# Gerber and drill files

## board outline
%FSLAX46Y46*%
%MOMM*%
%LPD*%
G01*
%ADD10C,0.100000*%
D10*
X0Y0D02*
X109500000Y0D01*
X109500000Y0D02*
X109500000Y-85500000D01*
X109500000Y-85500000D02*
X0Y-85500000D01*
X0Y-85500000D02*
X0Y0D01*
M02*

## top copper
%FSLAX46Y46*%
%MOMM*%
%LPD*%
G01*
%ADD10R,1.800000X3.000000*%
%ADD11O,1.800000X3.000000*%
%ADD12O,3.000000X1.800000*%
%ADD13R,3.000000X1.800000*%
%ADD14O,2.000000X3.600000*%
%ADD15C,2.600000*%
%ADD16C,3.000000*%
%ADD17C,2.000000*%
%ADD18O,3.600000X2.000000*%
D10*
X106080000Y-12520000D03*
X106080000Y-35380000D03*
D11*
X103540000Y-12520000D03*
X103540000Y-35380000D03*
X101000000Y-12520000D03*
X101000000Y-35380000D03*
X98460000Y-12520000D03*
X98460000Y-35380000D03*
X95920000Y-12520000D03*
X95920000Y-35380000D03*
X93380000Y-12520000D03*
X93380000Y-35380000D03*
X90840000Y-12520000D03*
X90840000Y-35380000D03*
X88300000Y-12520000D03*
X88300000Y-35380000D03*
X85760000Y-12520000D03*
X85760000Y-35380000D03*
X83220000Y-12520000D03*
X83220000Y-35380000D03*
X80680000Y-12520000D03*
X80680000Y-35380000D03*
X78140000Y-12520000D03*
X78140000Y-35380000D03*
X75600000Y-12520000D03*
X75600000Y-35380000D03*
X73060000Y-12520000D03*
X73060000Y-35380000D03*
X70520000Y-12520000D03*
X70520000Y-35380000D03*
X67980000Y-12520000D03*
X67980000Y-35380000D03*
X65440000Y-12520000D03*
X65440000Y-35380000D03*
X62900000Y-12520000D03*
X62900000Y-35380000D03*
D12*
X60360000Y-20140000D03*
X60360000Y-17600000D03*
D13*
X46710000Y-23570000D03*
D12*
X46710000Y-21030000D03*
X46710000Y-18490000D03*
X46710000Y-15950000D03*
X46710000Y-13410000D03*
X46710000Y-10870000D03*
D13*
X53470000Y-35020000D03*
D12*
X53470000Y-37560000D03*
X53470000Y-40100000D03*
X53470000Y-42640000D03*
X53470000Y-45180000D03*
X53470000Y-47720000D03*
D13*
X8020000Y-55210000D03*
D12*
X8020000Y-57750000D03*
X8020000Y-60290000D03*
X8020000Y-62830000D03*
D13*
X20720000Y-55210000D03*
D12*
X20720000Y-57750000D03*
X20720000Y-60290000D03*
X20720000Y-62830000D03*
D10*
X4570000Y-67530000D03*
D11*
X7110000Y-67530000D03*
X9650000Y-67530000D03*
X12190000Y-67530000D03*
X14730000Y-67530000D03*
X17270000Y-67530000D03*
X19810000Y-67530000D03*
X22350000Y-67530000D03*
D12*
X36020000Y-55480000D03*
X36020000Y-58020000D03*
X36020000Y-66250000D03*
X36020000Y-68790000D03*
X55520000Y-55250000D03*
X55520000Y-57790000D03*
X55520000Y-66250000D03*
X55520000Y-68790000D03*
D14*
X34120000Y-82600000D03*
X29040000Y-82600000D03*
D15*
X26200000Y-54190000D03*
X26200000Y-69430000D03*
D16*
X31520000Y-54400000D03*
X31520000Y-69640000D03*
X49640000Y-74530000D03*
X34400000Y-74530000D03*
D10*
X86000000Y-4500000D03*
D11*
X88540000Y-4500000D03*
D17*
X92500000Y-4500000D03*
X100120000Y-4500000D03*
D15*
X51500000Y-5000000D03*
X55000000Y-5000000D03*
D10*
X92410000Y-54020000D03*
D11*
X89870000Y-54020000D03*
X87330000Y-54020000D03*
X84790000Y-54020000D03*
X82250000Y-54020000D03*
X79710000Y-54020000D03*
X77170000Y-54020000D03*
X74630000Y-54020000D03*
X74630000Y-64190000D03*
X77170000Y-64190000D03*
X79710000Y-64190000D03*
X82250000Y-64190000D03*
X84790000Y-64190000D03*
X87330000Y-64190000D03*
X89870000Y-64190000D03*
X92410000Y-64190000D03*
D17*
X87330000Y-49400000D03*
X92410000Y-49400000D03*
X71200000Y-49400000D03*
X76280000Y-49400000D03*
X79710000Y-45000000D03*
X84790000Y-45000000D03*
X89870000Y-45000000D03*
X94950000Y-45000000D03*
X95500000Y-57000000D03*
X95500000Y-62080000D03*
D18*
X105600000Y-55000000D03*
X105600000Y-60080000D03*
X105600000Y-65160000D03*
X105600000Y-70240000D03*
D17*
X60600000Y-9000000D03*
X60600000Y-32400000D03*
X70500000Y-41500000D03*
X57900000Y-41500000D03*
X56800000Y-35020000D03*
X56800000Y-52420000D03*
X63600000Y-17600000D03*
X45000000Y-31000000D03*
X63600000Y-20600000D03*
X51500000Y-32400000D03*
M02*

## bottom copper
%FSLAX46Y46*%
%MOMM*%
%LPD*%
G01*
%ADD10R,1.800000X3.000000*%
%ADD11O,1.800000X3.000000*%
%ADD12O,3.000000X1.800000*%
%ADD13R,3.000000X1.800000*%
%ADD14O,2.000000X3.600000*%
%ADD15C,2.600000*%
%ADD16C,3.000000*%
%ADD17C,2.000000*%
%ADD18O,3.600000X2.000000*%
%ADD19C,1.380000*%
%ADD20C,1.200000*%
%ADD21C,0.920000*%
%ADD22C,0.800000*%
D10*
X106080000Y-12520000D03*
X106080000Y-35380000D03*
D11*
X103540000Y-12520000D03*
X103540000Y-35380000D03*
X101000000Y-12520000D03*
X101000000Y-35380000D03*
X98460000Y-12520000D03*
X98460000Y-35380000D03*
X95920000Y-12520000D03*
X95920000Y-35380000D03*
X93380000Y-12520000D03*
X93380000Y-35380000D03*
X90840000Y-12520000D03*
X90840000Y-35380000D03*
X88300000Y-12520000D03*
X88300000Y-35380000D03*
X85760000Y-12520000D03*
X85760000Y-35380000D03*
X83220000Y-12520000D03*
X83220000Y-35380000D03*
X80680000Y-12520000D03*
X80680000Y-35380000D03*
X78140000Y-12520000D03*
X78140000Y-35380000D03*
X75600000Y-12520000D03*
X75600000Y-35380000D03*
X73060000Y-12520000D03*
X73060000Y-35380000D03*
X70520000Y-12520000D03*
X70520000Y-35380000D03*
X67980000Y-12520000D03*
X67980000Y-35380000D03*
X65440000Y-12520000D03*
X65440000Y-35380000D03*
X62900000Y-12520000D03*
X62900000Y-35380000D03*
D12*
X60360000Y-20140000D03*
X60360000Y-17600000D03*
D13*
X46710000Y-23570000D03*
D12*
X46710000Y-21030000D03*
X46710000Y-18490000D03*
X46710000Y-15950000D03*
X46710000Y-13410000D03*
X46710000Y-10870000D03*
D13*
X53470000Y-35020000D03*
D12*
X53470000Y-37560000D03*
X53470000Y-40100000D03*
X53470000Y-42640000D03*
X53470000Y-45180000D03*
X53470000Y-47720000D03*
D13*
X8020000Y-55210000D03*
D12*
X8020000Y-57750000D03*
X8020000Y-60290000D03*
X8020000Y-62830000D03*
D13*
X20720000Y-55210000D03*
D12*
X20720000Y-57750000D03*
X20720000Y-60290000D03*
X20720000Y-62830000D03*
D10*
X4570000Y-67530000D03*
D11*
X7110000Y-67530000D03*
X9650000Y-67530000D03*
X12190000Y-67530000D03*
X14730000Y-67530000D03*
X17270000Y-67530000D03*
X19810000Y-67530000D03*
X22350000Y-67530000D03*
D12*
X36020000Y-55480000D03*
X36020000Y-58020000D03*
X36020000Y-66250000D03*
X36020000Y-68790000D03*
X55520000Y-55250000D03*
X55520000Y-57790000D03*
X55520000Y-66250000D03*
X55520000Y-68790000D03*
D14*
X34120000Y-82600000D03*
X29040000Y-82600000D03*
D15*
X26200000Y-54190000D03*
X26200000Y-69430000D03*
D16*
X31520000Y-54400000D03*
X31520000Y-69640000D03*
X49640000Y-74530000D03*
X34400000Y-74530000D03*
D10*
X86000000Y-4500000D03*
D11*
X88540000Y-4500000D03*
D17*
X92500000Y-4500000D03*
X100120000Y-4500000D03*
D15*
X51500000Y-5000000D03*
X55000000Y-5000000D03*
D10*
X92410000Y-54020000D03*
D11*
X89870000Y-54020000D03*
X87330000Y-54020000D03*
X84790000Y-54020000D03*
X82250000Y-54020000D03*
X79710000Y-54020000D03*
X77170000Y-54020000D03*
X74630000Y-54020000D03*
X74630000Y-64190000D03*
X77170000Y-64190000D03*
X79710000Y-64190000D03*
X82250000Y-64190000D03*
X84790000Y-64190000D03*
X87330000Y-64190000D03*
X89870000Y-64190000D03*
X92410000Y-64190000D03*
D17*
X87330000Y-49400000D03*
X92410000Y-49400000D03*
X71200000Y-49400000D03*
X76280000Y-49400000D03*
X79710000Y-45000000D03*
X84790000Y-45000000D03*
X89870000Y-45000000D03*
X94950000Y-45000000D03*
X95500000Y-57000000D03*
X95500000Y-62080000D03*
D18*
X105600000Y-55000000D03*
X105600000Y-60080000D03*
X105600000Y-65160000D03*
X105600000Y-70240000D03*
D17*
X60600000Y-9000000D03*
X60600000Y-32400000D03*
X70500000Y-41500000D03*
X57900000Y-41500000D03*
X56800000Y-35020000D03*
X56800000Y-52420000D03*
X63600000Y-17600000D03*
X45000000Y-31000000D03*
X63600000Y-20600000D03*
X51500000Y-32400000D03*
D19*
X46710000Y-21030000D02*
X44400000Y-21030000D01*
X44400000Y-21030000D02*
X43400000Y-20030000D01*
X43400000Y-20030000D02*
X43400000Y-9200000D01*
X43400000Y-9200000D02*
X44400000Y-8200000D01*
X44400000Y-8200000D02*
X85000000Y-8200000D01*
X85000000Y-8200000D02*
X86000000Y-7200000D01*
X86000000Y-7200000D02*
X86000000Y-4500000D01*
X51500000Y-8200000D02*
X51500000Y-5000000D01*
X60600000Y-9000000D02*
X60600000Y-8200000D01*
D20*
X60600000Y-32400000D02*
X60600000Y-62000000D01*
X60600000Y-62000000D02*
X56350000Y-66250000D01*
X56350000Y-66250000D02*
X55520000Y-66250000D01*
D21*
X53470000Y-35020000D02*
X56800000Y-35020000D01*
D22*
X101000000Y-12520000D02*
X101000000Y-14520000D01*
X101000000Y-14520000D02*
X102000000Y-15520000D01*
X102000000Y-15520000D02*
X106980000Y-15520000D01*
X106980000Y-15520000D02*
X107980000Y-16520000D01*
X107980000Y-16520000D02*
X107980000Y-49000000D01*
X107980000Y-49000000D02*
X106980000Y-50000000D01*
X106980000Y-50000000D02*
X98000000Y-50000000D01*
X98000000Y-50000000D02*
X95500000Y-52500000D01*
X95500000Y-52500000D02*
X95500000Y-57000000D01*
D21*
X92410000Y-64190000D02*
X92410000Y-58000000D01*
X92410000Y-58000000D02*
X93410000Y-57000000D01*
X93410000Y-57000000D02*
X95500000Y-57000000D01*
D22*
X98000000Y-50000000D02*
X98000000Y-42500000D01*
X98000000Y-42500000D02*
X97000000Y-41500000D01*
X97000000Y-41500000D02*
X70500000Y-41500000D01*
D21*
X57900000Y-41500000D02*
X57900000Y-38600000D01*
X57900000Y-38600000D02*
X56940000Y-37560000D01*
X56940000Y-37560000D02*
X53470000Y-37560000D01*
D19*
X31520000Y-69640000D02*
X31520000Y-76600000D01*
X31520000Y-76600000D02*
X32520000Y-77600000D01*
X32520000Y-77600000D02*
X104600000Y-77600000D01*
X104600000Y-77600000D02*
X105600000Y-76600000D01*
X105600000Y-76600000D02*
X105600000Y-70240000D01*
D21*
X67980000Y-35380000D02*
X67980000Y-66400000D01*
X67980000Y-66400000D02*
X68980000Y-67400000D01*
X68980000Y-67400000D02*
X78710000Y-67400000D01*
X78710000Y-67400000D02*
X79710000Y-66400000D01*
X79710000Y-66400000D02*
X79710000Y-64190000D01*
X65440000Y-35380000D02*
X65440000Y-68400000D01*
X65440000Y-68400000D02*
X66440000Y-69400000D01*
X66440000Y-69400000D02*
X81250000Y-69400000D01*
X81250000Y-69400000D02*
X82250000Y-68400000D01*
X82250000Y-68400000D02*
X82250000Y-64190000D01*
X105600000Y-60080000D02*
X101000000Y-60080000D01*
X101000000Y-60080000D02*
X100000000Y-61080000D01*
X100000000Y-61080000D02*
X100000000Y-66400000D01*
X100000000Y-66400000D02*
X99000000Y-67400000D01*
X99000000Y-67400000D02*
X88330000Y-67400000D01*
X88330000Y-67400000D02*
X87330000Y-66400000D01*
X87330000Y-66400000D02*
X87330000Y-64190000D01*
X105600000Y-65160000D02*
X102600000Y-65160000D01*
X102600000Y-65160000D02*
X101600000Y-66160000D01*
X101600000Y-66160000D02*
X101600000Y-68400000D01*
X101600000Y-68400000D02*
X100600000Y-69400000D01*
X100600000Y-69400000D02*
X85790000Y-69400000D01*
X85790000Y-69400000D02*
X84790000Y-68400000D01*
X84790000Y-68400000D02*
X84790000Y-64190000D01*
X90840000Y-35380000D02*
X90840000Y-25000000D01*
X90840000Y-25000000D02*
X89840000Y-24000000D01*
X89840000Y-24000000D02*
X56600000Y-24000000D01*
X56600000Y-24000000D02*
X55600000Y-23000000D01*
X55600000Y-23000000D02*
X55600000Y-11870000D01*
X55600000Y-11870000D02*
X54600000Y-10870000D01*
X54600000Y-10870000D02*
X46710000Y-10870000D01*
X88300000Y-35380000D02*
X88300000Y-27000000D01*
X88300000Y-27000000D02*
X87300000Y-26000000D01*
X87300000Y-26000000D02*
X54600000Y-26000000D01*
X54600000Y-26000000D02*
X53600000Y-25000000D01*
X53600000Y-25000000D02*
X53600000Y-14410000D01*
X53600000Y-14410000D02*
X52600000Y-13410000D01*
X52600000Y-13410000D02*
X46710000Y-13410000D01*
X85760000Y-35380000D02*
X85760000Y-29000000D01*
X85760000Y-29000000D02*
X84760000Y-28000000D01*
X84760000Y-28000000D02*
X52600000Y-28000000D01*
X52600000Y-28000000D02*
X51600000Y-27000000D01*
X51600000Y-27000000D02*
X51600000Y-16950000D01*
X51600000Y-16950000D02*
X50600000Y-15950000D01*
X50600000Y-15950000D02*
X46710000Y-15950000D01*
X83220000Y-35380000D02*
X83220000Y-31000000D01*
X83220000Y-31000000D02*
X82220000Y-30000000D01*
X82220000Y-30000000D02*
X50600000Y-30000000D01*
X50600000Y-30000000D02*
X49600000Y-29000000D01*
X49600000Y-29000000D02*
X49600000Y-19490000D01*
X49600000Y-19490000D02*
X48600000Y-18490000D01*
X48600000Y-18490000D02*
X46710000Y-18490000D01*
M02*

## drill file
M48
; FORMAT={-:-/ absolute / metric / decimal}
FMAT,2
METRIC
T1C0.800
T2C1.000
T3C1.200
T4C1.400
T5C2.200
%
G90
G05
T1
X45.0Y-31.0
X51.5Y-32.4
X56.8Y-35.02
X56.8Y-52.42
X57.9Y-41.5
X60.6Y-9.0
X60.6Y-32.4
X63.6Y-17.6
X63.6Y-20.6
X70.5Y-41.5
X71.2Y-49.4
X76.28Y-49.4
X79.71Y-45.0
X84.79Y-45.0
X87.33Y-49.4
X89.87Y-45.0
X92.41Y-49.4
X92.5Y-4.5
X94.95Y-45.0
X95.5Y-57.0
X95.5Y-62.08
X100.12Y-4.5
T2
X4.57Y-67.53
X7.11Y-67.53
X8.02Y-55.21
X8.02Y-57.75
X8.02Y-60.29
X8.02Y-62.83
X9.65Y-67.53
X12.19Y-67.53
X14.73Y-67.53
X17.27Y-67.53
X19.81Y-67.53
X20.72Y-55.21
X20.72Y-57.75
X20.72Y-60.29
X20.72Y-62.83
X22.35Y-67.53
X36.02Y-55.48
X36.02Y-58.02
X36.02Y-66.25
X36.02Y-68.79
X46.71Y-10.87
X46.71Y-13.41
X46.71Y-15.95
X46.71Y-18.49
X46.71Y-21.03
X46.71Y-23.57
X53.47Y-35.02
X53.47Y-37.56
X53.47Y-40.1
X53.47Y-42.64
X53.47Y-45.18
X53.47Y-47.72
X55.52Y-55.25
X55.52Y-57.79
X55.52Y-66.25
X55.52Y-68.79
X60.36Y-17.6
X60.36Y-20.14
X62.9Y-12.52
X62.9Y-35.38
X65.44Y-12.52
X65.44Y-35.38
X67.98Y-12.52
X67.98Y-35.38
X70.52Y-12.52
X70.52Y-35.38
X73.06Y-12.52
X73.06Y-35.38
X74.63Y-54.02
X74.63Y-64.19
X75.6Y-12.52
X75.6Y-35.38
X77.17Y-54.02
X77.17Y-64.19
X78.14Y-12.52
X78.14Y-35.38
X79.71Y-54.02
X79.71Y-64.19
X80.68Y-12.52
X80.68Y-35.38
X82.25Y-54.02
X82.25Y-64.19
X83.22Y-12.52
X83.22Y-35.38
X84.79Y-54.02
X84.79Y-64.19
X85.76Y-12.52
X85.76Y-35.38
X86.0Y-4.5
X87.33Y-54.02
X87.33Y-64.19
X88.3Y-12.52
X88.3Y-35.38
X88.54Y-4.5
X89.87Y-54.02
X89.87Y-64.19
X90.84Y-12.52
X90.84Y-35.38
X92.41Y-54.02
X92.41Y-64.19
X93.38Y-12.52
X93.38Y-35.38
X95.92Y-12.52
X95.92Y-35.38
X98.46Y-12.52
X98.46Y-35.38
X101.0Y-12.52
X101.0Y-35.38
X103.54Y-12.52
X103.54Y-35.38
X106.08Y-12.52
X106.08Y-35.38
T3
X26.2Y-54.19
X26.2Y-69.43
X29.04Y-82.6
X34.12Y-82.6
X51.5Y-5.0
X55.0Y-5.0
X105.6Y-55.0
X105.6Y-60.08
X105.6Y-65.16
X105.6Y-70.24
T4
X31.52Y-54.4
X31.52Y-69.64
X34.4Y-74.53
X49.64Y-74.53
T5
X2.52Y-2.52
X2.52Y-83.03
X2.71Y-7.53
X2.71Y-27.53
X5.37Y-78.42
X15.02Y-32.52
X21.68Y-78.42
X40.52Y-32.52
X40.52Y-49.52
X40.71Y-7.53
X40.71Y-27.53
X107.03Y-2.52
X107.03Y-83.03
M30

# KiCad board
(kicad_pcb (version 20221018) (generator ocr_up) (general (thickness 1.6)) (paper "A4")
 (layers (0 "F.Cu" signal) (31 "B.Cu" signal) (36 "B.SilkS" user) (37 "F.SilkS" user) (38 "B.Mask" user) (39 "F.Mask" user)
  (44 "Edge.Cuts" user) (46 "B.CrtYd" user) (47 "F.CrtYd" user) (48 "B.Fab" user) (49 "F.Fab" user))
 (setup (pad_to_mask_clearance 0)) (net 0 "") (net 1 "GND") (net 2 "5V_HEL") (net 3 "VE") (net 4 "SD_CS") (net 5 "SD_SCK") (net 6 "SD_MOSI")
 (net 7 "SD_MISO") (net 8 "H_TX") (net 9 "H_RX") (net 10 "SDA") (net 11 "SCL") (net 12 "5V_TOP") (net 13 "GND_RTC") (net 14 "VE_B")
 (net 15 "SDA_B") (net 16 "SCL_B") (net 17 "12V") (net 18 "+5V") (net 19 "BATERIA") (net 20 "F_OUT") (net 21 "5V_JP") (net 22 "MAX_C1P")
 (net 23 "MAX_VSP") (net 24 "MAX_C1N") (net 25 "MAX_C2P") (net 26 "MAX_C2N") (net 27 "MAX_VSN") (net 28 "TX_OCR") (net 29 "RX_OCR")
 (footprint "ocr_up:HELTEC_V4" (layer "F.Cu") (at 106.08 12.52)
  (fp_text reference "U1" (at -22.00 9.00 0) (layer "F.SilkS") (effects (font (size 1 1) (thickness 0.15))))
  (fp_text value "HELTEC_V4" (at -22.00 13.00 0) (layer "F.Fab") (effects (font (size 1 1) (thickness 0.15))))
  (pad "A1" thru_hole rect (at -0.0 0) (size 1.8 3.0) (drill 1.0) (layers "*.Cu" "*.Mask") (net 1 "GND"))
  (pad "B1" thru_hole rect (at -0.0 22.86) (size 1.8 3.0) (drill 1.0) (layers "*.Cu" "*.Mask"))
  (pad "A2" thru_hole oval (at -2.54 0) (size 1.8 3.0) (drill 1.0) (layers "*.Cu" "*.Mask") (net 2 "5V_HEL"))
  (pad "B2" thru_hole oval (at -2.54 22.86) (size 1.8 3.0) (drill 1.0) (layers "*.Cu" "*.Mask"))
  (pad "A3" thru_hole oval (at -5.08 0) (size 1.8 3.0) (drill 1.0) (layers "*.Cu" "*.Mask") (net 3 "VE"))
  (pad "B3" thru_hole oval (at -5.08 22.86) (size 1.8 3.0) (drill 1.0) (layers "*.Cu" "*.Mask"))
  (pad "A4" thru_hole oval (at -7.62 0) (size 1.8 3.0) (drill 1.0) (layers "*.Cu" "*.Mask") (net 3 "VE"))
  (pad "B4" thru_hole oval (at -7.62 22.86) (size 1.8 3.0) (drill 1.0) (layers "*.Cu" "*.Mask"))
  (pad "A5" thru_hole oval (at -10.16 0) (size 1.8 3.0) (drill 1.0) (layers "*.Cu" "*.Mask"))
  (pad "B5" thru_hole oval (at -10.16 22.86) (size 1.8 3.0) (drill 1.0) (layers "*.Cu" "*.Mask"))
  (pad "A6" thru_hole oval (at -12.7 0) (size 1.8 3.0) (drill 1.0) (layers "*.Cu" "*.Mask"))
  (pad "B6" thru_hole oval (at -12.7 22.86) (size 1.8 3.0) (drill 1.0) (layers "*.Cu" "*.Mask"))
  (pad "A7" thru_hole oval (at -15.24 0) (size 1.8 3.0) (drill 1.0) (layers "*.Cu" "*.Mask"))
  (pad "B7" thru_hole oval (at -15.24 22.86) (size 1.8 3.0) (drill 1.0) (layers "*.Cu" "*.Mask") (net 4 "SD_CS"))
  (pad "A8" thru_hole oval (at -17.78 0) (size 1.8 3.0) (drill 1.0) (layers "*.Cu" "*.Mask"))
  (pad "B8" thru_hole oval (at -17.78 22.86) (size 1.8 3.0) (drill 1.0) (layers "*.Cu" "*.Mask") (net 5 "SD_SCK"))
  (pad "A9" thru_hole oval (at -20.32 0) (size 1.8 3.0) (drill 1.0) (layers "*.Cu" "*.Mask"))
  (pad "B9" thru_hole oval (at -20.32 22.86) (size 1.8 3.0) (drill 1.0) (layers "*.Cu" "*.Mask") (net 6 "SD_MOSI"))
  (pad "A10" thru_hole oval (at -22.86 0) (size 1.8 3.0) (drill 1.0) (layers "*.Cu" "*.Mask"))
  (pad "B10" thru_hole oval (at -22.86 22.86) (size 1.8 3.0) (drill 1.0) (layers "*.Cu" "*.Mask") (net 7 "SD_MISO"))
  (pad "A11" thru_hole oval (at -25.4 0) (size 1.8 3.0) (drill 1.0) (layers "*.Cu" "*.Mask"))
  (pad "B11" thru_hole oval (at -25.4 22.86) (size 1.8 3.0) (drill 1.0) (layers "*.Cu" "*.Mask"))
  (pad "A12" thru_hole oval (at -27.94 0) (size 1.8 3.0) (drill 1.0) (layers "*.Cu" "*.Mask"))
  (pad "B12" thru_hole oval (at -27.94 22.86) (size 1.8 3.0) (drill 1.0) (layers "*.Cu" "*.Mask"))
  (pad "A13" thru_hole oval (at -30.48 0) (size 1.8 3.0) (drill 1.0) (layers "*.Cu" "*.Mask"))
  (pad "B13" thru_hole oval (at -30.48 22.86) (size 1.8 3.0) (drill 1.0) (layers "*.Cu" "*.Mask"))
  (pad "A14" thru_hole oval (at -33.02 0) (size 1.8 3.0) (drill 1.0) (layers "*.Cu" "*.Mask"))
  (pad "B14" thru_hole oval (at -33.02 22.86) (size 1.8 3.0) (drill 1.0) (layers "*.Cu" "*.Mask"))
  (pad "A15" thru_hole oval (at -35.56 0) (size 1.8 3.0) (drill 1.0) (layers "*.Cu" "*.Mask"))
  (pad "B15" thru_hole oval (at -35.56 22.86) (size 1.8 3.0) (drill 1.0) (layers "*.Cu" "*.Mask"))
  (pad "A16" thru_hole oval (at -38.1 0) (size 1.8 3.0) (drill 1.0) (layers "*.Cu" "*.Mask"))
  (pad "B16" thru_hole oval (at -38.1 22.86) (size 1.8 3.0) (drill 1.0) (layers "*.Cu" "*.Mask") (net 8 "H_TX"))
  (pad "A17" thru_hole oval (at -40.64 0) (size 1.8 3.0) (drill 1.0) (layers "*.Cu" "*.Mask"))
  (pad "B17" thru_hole oval (at -40.64 22.86) (size 1.8 3.0) (drill 1.0) (layers "*.Cu" "*.Mask") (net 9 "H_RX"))
  (pad "A18" thru_hole oval (at -43.18 0) (size 1.8 3.0) (drill 1.0) (layers "*.Cu" "*.Mask"))
  (pad "B18" thru_hole oval (at -43.18 22.86) (size 1.8 3.0) (drill 1.0) (layers "*.Cu" "*.Mask"))
  (pad "AUX17" thru_hole oval (at -45.72 7.619999999999999) (size 3.0 1.8) (drill 1.0) (layers "*.Cu" "*.Mask") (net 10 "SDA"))
  (pad "AUX18" thru_hole oval (at -45.72 5.08) (size 3.0 1.8) (drill 1.0) (layers "*.Cu" "*.Mask") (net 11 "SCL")))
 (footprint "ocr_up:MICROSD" (layer "F.Cu") (at 0.66 5.48)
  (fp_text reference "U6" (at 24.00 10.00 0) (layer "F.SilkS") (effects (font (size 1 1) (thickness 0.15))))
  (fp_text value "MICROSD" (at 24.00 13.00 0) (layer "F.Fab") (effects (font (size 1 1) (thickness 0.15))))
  (pad "1" thru_hole rect (at 46.05 18.09) (size 3.0 1.8) (drill 1.0) (layers "*.Cu" "*.Mask") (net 1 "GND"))
  (pad "2" thru_hole oval (at 46.05 15.55) (size 3.0 1.8) (drill 1.0) (layers "*.Cu" "*.Mask") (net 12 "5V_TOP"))
  (pad "3" thru_hole oval (at 46.05 13.01) (size 3.0 1.8) (drill 1.0) (layers "*.Cu" "*.Mask") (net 7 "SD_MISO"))
  (pad "4" thru_hole oval (at 46.05 10.469999999999999) (size 3.0 1.8) (drill 1.0) (layers "*.Cu" "*.Mask") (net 6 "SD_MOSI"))
  (pad "5" thru_hole oval (at 46.05 7.93) (size 3.0 1.8) (drill 1.0) (layers "*.Cu" "*.Mask") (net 5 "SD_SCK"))
  (pad "6" thru_hole oval (at 46.05 5.390000000000001) (size 3.0 1.8) (drill 1.0) (layers "*.Cu" "*.Mask") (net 4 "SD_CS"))
  (pad "" np_thru_hole circle (at 2.05 2.05) (size 2.2 2.2) (drill 2.2) (layers "*.Cu" "*.Mask"))
  (pad "" np_thru_hole circle (at 40.05 2.05) (size 2.2 2.2) (drill 2.2) (layers "*.Cu" "*.Mask"))
  (pad "" np_thru_hole circle (at 2.05 22.05) (size 2.2 2.2) (drill 2.2) (layers "*.Cu" "*.Mask"))
  (pad "" np_thru_hole circle (at 40.05 22.05) (size 2.2 2.2) (drill 2.2) (layers "*.Cu" "*.Mask")))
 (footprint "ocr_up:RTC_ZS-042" (layer "F.Cu") (at 53.47 35.02)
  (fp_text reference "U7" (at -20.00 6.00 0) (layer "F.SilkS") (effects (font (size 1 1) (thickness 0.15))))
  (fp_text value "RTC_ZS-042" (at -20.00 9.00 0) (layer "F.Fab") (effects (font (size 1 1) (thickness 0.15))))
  (pad "1" thru_hole rect (at 0 0.0) (size 3.0 1.8) (drill 1.0) (layers "*.Cu" "*.Mask") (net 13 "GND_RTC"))
  (pad "2" thru_hole oval (at 0 2.54) (size 3.0 1.8) (drill 1.0) (layers "*.Cu" "*.Mask") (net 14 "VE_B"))
  (pad "3" thru_hole oval (at 0 5.08) (size 3.0 1.8) (drill 1.0) (layers "*.Cu" "*.Mask") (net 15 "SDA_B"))
  (pad "4" thru_hole oval (at 0 7.62) (size 3.0 1.8) (drill 1.0) (layers "*.Cu" "*.Mask") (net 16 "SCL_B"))
  (pad "5" thru_hole oval (at 0 10.16) (size 3.0 1.8) (drill 1.0) (layers "*.Cu" "*.Mask"))
  (pad "6" thru_hole oval (at 0 12.7) (size 3.0 1.8) (drill 1.0) (layers "*.Cu" "*.Mask"))
  (pad "" np_thru_hole circle (at -38.45 -2.5) (size 2.2 2.2) (drill 2.2) (layers "*.Cu" "*.Mask"))
  (pad "" np_thru_hole circle (at -12.949999999999996 -2.5) (size 2.2 2.2) (drill 2.2) (layers "*.Cu" "*.Mask"))
  (pad "" np_thru_hole circle (at -12.949999999999996 14.5) (size 2.2 2.2) (drill 2.2) (layers "*.Cu" "*.Mask")))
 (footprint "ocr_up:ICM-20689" (layer "F.Cu") (at 8.02 55.21)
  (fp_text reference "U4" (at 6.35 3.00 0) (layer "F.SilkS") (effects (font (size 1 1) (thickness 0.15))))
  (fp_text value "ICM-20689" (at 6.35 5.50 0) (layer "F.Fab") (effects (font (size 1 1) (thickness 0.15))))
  (pad "1" thru_hole rect (at 0 0.0) (size 3.0 1.8) (drill 1.0) (layers "*.Cu" "*.Mask") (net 14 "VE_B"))
  (pad "2" thru_hole oval (at 0 2.54) (size 3.0 1.8) (drill 1.0) (layers "*.Cu" "*.Mask") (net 1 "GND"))
  (pad "3" thru_hole oval (at 0 5.08) (size 3.0 1.8) (drill 1.0) (layers "*.Cu" "*.Mask") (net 16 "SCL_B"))
  (pad "4" thru_hole oval (at 0 7.62) (size 3.0 1.8) (drill 1.0) (layers "*.Cu" "*.Mask") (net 15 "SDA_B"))
  (pad "5" thru_hole rect (at 12.7 0.0) (size 3.0 1.8) (drill 1.0) (layers "*.Cu" "*.Mask"))
  (pad "6" thru_hole oval (at 12.7 2.54) (size 3.0 1.8) (drill 1.0) (layers "*.Cu" "*.Mask"))
  (pad "7" thru_hole oval (at 12.7 5.08) (size 3.0 1.8) (drill 1.0) (layers "*.Cu" "*.Mask"))
  (pad "8" thru_hole oval (at 12.7 7.62) (size 3.0 1.8) (drill 1.0) (layers "*.Cu" "*.Mask") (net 14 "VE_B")))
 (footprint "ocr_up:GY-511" (layer "F.Cu") (at 4.57 67.53)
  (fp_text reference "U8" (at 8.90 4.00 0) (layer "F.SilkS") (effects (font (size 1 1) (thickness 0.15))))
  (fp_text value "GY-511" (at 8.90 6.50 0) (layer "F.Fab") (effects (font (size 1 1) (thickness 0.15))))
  (pad "1" thru_hole rect (at 0.0 0) (size 1.8 3.0) (drill 1.0) (layers "*.Cu" "*.Mask"))
  (pad "2" thru_hole oval (at 2.54 0) (size 1.8 3.0) (drill 1.0) (layers "*.Cu" "*.Mask"))
  (pad "3" thru_hole oval (at 5.08 0) (size 1.8 3.0) (drill 1.0) (layers "*.Cu" "*.Mask"))
  (pad "4" thru_hole oval (at 7.62 0) (size 1.8 3.0) (drill 1.0) (layers "*.Cu" "*.Mask") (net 15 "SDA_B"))
  (pad "5" thru_hole oval (at 10.16 0) (size 1.8 3.0) (drill 1.0) (layers "*.Cu" "*.Mask") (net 16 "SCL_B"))
  (pad "6" thru_hole oval (at 12.7 0) (size 1.8 3.0) (drill 1.0) (layers "*.Cu" "*.Mask") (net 1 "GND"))
  (pad "7" thru_hole oval (at 15.24 0) (size 1.8 3.0) (drill 1.0) (layers "*.Cu" "*.Mask") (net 14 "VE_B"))
  (pad "8" thru_hole oval (at 17.78 0) (size 1.8 3.0) (drill 1.0) (layers "*.Cu" "*.Mask"))
  (pad "" np_thru_hole circle (at 0.7999999999999998 10.89) (size 2.2 2.2) (drill 2.2) (layers "*.Cu" "*.Mask"))
  (pad "" np_thru_hole circle (at 17.11 10.89) (size 2.2 2.2) (drill 2.2) (layers "*.Cu" "*.Mask")))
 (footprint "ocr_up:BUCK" (layer "F.Cu") (at 36.02 55.48)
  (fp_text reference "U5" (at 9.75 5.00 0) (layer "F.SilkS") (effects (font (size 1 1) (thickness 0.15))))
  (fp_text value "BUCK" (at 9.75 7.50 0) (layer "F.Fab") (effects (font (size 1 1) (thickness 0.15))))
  (pad "1" thru_hole oval (at 0 0) (size 3.0 1.8) (drill 1.0) (layers "*.Cu" "*.Mask"))
  (pad "2" thru_hole oval (at 0 2.54) (size 3.0 1.8) (drill 1.0) (layers "*.Cu" "*.Mask"))
  (pad "3" thru_hole oval (at 0 10.77) (size 3.0 1.8) (drill 1.0) (layers "*.Cu" "*.Mask") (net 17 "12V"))
  (pad "4" thru_hole oval (at 0 13.31) (size 3.0 1.8) (drill 1.0) (layers "*.Cu" "*.Mask"))
  (pad "5" thru_hole oval (at 19.5 -0.23) (size 3.0 1.8) (drill 1.0) (layers "*.Cu" "*.Mask"))
  (pad "6" thru_hole oval (at 19.5 2.31) (size 3.0 1.8) (drill 1.0) (layers "*.Cu" "*.Mask") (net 1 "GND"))
  (pad "7" thru_hole oval (at 19.5 10.77) (size 3.0 1.8) (drill 1.0) (layers "*.Cu" "*.Mask") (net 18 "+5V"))
  (pad "8" thru_hole oval (at 19.5 13.31) (size 3.0 1.8) (drill 1.0) (layers "*.Cu" "*.Mask")))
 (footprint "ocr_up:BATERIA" (layer "F.Cu") (at 34.12 82.6)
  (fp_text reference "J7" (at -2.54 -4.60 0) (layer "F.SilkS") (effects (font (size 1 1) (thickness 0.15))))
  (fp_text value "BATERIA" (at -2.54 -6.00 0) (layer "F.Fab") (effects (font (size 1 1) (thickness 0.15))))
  (pad "1" thru_hole oval (at -0.0 0) (size 2.0 3.6) (drill 1.2) (layers "*.Cu" "*.Mask") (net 1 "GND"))
  (pad "2" thru_hole oval (at -5.08 0) (size 2.0 3.6) (drill 1.2) (layers "*.Cu" "*.Mask") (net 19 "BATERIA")))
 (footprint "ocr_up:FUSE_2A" (layer "F.Cu") (at 26.2 54.19)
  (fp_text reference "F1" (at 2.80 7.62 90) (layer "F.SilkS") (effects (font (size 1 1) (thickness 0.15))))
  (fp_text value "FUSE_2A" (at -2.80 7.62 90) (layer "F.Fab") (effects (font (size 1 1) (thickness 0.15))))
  (pad "1" thru_hole circle (at 0 0) (size 2.6 2.6) (drill 1.2) (layers "*.Cu" "*.Mask") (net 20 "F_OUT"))
  (pad "2" thru_hole circle (at 0 15.24) (size 2.6 2.6) (drill 1.2) (layers "*.Cu" "*.Mask") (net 19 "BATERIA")))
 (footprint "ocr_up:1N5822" (layer "F.Cu") (at 31.52 54.4)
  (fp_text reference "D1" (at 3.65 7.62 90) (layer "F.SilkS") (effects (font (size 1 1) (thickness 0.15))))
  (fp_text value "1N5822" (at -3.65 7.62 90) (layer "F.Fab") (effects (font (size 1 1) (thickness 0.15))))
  (pad "1" thru_hole circle (at 0 0) (size 3.0 3.0) (drill 1.4) (layers "*.Cu" "*.Mask") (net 20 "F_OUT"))
  (pad "2" thru_hole circle (at 0 15.24) (size 3.0 3.0) (drill 1.4) (layers "*.Cu" "*.Mask") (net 17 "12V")))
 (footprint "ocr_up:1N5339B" (layer "F.Cu") (at 49.64 74.53)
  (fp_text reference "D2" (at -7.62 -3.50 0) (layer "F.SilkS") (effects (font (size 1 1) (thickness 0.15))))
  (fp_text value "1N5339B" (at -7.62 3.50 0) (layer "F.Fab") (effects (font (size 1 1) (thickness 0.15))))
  (pad "1" thru_hole circle (at 0 0) (size 3.0 3.0) (drill 1.4) (layers "*.Cu" "*.Mask") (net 18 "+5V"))
  (pad "2" thru_hole circle (at -15.24 0) (size 3.0 3.0) (drill 1.4) (layers "*.Cu" "*.Mask") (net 1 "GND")))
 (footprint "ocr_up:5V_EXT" (layer "F.Cu") (at 86.0 4.5)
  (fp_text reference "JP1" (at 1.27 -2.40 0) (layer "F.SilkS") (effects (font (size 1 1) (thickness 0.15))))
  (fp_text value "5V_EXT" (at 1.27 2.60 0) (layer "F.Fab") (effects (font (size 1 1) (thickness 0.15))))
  (pad "1" thru_hole rect (at 0 0) (size 1.8 3.0) (drill 1.0) (layers "*.Cu" "*.Mask") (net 12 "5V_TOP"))
  (pad "2" thru_hole oval (at 2.54 0) (size 1.8 3.0) (drill 1.0) (layers "*.Cu" "*.Mask") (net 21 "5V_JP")))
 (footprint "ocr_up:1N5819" (layer "F.Cu") (at 92.5 4.5)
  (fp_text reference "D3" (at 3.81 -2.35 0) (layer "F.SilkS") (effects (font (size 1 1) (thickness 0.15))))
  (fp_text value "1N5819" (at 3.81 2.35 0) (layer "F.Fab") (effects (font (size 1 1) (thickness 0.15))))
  (pad "1" thru_hole circle (at 0 0) (size 2.0 2.0) (drill 0.8) (layers "*.Cu" "*.Mask") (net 21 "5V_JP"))
  (pad "2" thru_hole circle (at 7.62 0) (size 2.0 2.0) (drill 0.8) (layers "*.Cu" "*.Mask") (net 2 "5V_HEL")))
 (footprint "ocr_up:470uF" (layer "F.Cu") (at 51.5 5.0)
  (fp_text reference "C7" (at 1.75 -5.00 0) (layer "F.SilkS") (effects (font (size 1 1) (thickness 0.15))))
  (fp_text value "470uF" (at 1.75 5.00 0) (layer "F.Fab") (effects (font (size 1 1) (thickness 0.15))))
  (pad "1" thru_hole circle (at 0 0) (size 2.6 2.6) (drill 1.2) (layers "*.Cu" "*.Mask") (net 12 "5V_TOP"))
  (pad "2" thru_hole circle (at 3.5 0) (size 2.6 2.6) (drill 1.2) (layers "*.Cu" "*.Mask") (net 1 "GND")))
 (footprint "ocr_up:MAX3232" (layer "F.Cu") (at 74.63 64.19)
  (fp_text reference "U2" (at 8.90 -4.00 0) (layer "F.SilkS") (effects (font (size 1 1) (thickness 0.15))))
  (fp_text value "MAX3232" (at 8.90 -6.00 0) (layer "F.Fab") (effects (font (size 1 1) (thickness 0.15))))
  (pad "1" thru_hole rect (at 17.78 -10.17) (size 1.8 3.0) (drill 1.0) (layers "*.Cu" "*.Mask") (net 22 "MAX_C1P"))
  (pad "2" thru_hole oval (at 15.24 -10.17) (size 1.8 3.0) (drill 1.0) (layers "*.Cu" "*.Mask") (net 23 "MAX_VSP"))
  (pad "3" thru_hole oval (at 12.7 -10.17) (size 1.8 3.0) (drill 1.0) (layers "*.Cu" "*.Mask") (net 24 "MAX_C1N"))
  (pad "4" thru_hole oval (at 10.16 -10.17) (size 1.8 3.0) (drill 1.0) (layers "*.Cu" "*.Mask") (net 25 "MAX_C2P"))
  (pad "5" thru_hole oval (at 7.62 -10.17) (size 1.8 3.0) (drill 1.0) (layers "*.Cu" "*.Mask") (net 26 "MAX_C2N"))
  (pad "6" thru_hole oval (at 5.08 -10.17) (size 1.8 3.0) (drill 1.0) (layers "*.Cu" "*.Mask") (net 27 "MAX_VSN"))
  (pad "7" thru_hole oval (at 2.54 -10.17) (size 1.8 3.0) (drill 1.0) (layers "*.Cu" "*.Mask"))
  (pad "8" thru_hole oval (at 0.0 -10.17) (size 1.8 3.0) (drill 1.0) (layers "*.Cu" "*.Mask"))
  (pad "9" thru_hole oval (at 0.0 0.0) (size 1.8 3.0) (drill 1.0) (layers "*.Cu" "*.Mask"))
  (pad "10" thru_hole oval (at 2.54 0.0) (size 1.8 3.0) (drill 1.0) (layers "*.Cu" "*.Mask") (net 1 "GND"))
  (pad "11" thru_hole oval (at 5.08 0.0) (size 1.8 3.0) (drill 1.0) (layers "*.Cu" "*.Mask") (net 8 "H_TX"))
  (pad "12" thru_hole oval (at 7.62 0.0) (size 1.8 3.0) (drill 1.0) (layers "*.Cu" "*.Mask") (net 9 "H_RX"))
  (pad "13" thru_hole oval (at 10.16 0.0) (size 1.8 3.0) (drill 1.0) (layers "*.Cu" "*.Mask") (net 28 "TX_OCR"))
  (pad "14" thru_hole oval (at 12.7 0.0) (size 1.8 3.0) (drill 1.0) (layers "*.Cu" "*.Mask") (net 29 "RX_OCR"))
  (pad "15" thru_hole oval (at 15.24 0.0) (size 1.8 3.0) (drill 1.0) (layers "*.Cu" "*.Mask") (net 1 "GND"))
  (pad "16" thru_hole oval (at 17.78 0.0) (size 1.8 3.0) (drill 1.0) (layers "*.Cu" "*.Mask") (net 3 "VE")))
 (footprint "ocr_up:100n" (layer "F.Cu") (at 87.33 49.4)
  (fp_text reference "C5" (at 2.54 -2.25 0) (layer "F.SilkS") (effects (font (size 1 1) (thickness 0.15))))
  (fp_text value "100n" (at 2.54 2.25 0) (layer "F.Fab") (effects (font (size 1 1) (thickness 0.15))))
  (pad "1" thru_hole circle (at 0 0) (size 2.0 2.0) (drill 0.8) (layers "*.Cu" "*.Mask") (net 24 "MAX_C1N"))
  (pad "2" thru_hole circle (at 5.08 0) (size 2.0 2.0) (drill 0.8) (layers "*.Cu" "*.Mask") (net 22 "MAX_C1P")))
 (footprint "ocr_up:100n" (layer "F.Cu") (at 71.2 49.4)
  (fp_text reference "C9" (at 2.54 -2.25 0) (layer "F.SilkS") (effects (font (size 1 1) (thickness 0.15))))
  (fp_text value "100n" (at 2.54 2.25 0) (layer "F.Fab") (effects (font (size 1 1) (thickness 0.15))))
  (pad "1" thru_hole circle (at 0 0) (size 2.0 2.0) (drill 0.8) (layers "*.Cu" "*.Mask") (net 1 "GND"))
  (pad "2" thru_hole circle (at 5.08 0) (size 2.0 2.0) (drill 0.8) (layers "*.Cu" "*.Mask") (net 27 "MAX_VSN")))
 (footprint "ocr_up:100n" (layer "F.Cu") (at 79.71 45.0)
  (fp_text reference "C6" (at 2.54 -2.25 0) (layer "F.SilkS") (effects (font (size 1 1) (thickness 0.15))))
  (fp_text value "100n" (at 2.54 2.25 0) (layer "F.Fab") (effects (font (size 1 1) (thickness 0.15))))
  (pad "1" thru_hole circle (at 0 0) (size 2.0 2.0) (drill 0.8) (layers "*.Cu" "*.Mask") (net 26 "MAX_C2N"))
  (pad "2" thru_hole circle (at 5.08 0) (size 2.0 2.0) (drill 0.8) (layers "*.Cu" "*.Mask") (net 25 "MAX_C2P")))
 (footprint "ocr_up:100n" (layer "F.Cu") (at 89.87 45.0)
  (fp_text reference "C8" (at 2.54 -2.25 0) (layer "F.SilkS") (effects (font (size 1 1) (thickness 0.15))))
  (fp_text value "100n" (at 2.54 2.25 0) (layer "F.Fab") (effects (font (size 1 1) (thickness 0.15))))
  (pad "1" thru_hole circle (at 0 0) (size 2.0 2.0) (drill 0.8) (layers "*.Cu" "*.Mask") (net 23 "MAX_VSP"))
  (pad "2" thru_hole circle (at 5.08 0) (size 2.0 2.0) (drill 0.8) (layers "*.Cu" "*.Mask") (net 1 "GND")))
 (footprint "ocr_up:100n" (layer "F.Cu") (at 95.5 57.0)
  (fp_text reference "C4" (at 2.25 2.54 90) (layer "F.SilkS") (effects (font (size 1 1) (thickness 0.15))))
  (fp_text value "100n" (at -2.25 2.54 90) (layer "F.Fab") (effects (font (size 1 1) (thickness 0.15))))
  (pad "1" thru_hole circle (at 0 0) (size 2.0 2.0) (drill 0.8) (layers "*.Cu" "*.Mask") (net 3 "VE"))
  (pad "2" thru_hole circle (at 0 5.08) (size 2.0 2.0) (drill 0.8) (layers "*.Cu" "*.Mask") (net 1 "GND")))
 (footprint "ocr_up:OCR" (layer "F.Cu") (at 105.6 55.0)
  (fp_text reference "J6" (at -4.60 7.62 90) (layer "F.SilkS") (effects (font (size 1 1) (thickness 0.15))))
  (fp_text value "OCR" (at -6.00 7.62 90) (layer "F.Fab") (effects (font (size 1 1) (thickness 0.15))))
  (pad "1" thru_hole oval (at 0 0.0) (size 3.6 2.0) (drill 1.2) (layers "*.Cu" "*.Mask") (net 1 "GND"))
  (pad "2" thru_hole oval (at 0 5.08) (size 3.6 2.0) (drill 1.2) (layers "*.Cu" "*.Mask") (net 29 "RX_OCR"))
  (pad "3" thru_hole oval (at 0 10.16) (size 3.6 2.0) (drill 1.2) (layers "*.Cu" "*.Mask") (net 28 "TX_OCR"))
  (pad "4" thru_hole oval (at 0 15.24) (size 3.6 2.0) (drill 1.2) (layers "*.Cu" "*.Mask") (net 17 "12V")))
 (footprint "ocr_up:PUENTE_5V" (layer "F.Cu") (at 60.6 9.0)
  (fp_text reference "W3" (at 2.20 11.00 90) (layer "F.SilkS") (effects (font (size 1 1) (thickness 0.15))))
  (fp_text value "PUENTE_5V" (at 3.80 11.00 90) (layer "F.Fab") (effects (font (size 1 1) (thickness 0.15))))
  (pad "1" thru_hole circle (at 0 0) (size 2.0 2.0) (drill 0.8) (layers "*.Cu" "*.Mask") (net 12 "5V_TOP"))
  (pad "2" thru_hole circle (at 0 23.4) (size 2.0 2.0) (drill 0.8) (layers "*.Cu" "*.Mask") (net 18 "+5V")))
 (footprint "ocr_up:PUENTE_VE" (layer "F.Cu") (at 70.5 41.5)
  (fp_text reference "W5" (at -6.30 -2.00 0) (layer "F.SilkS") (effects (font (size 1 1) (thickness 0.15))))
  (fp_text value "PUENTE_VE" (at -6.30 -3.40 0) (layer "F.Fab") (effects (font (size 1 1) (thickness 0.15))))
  (pad "1" thru_hole circle (at 0 0) (size 2.0 2.0) (drill 0.8) (layers "*.Cu" "*.Mask") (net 3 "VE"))
  (pad "2" thru_hole circle (at -12.600000000000001 0) (size 2.0 2.0) (drill 0.8) (layers "*.Cu" "*.Mask") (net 14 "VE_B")))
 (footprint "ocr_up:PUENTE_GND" (layer "F.Cu") (at 56.8 35.02)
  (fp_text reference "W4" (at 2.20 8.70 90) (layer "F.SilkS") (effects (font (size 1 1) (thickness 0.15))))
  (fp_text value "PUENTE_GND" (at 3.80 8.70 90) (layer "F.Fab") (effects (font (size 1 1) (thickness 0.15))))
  (pad "1" thru_hole circle (at 0 0) (size 2.0 2.0) (drill 0.8) (layers "*.Cu" "*.Mask") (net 13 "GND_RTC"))
  (pad "2" thru_hole circle (at 0 17.4) (size 2.0 2.0) (drill 0.8) (layers "*.Cu" "*.Mask") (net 1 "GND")))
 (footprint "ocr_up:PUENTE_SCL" (layer "F.Cu") (at 63.6 17.6)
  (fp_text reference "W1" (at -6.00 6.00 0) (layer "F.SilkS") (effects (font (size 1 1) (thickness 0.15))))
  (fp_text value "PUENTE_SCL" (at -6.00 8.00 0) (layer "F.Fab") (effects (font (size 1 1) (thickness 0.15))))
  (pad "1" thru_hole circle (at 0 0) (size 2.0 2.0) (drill 0.8) (layers "*.Cu" "*.Mask") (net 11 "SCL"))
  (pad "2" thru_hole circle (at -18.6 13.399999999999999) (size 2.0 2.0) (drill 0.8) (layers "*.Cu" "*.Mask") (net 16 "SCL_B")))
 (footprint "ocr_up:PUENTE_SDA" (layer "F.Cu") (at 63.6 20.6)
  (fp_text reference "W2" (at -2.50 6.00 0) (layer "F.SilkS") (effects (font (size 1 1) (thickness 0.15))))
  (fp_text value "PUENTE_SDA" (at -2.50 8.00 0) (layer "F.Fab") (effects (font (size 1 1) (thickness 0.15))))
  (pad "1" thru_hole circle (at 0 0) (size 2.0 2.0) (drill 0.8) (layers "*.Cu" "*.Mask") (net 10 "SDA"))
  (pad "2" thru_hole circle (at -12.100000000000001 11.799999999999997) (size 2.0 2.0) (drill 0.8) (layers "*.Cu" "*.Mask") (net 15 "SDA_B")))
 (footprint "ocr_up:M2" (layer "F.Cu") (at 2.52 2.52)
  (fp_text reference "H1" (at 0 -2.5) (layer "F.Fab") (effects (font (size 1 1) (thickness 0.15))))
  (pad "" np_thru_hole circle (at 0 0) (size 2.2 2.2) (drill 2.2) (layers "*.Cu" "*.Mask")))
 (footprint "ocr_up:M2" (layer "F.Cu") (at 107.03 2.52)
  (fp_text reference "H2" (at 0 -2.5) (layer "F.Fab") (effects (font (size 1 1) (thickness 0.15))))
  (pad "" np_thru_hole circle (at 0 0) (size 2.2 2.2) (drill 2.2) (layers "*.Cu" "*.Mask")))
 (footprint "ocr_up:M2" (layer "F.Cu") (at 2.52 83.03)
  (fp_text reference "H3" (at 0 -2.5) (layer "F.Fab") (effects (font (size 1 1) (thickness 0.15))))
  (pad "" np_thru_hole circle (at 0 0) (size 2.2 2.2) (drill 2.2) (layers "*.Cu" "*.Mask")))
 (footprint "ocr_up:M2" (layer "F.Cu") (at 107.03 83.03)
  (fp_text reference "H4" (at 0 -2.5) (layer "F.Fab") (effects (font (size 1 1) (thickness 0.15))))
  (pad "" np_thru_hole circle (at 0 0) (size 2.2 2.2) (drill 2.2) (layers "*.Cu" "*.Mask")))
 (segment locked (start 46.709999999999994 21.03) (end 44.4 21.03) (width 1.38) (layer "B.Cu") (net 12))
 (segment locked (start 44.4 21.03) (end 43.4 20.03) (width 1.38) (layer "B.Cu") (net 12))
 (segment locked (start 43.4 20.03) (end 43.4 9.2) (width 1.38) (layer "B.Cu") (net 12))
 (segment locked (start 43.4 9.2) (end 44.4 8.2) (width 1.38) (layer "B.Cu") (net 12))
 (segment locked (start 44.4 8.2) (end 85.0 8.2) (width 1.38) (layer "B.Cu") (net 12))
 (segment locked (start 85.0 8.2) (end 86.0 7.2) (width 1.38) (layer "B.Cu") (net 12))
 (segment locked (start 86.0 7.2) (end 86.0 4.5) (width 1.38) (layer "B.Cu") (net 12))
 (segment locked (start 51.5 8.2) (end 51.5 5.0) (width 1.38) (layer "B.Cu") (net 12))
 (segment locked (start 60.6 9.0) (end 60.6 8.2) (width 1.38) (layer "B.Cu") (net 12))
 (segment locked (start 60.6 32.4) (end 60.6 62.0) (width 1.2) (layer "B.Cu") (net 18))
 (segment locked (start 60.6 62.0) (end 56.35 66.25) (width 1.2) (layer "B.Cu") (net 18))
 (segment locked (start 56.35 66.25) (end 55.52 66.25) (width 1.2) (layer "B.Cu") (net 18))
 (segment locked (start 53.47 35.02) (end 56.8 35.02) (width 0.92) (layer "B.Cu") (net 13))
 (segment locked (start 101.0 12.52) (end 101.0 14.52) (width 0.8) (layer "B.Cu") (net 3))
 (segment locked (start 101.0 14.52) (end 102.0 15.52) (width 0.8) (layer "B.Cu") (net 3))
 (segment locked (start 102.0 15.52) (end 106.98 15.52) (width 0.8) (layer "B.Cu") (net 3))
 (segment locked (start 106.98 15.52) (end 107.98 16.52) (width 0.8) (layer "B.Cu") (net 3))
 (segment locked (start 107.98 16.52) (end 107.98 49.0) (width 0.8) (layer "B.Cu") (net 3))
 (segment locked (start 107.98 49.0) (end 106.98 50.0) (width 0.8) (layer "B.Cu") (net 3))
 (segment locked (start 106.98 50.0) (end 98.0 50.0) (width 0.8) (layer "B.Cu") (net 3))
 (segment locked (start 98.0 50.0) (end 95.5 52.5) (width 0.8) (layer "B.Cu") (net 3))
 (segment locked (start 95.5 52.5) (end 95.5 57.0) (width 0.8) (layer "B.Cu") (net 3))
 (segment locked (start 92.41 64.19) (end 92.41 58.0) (width 0.92) (layer "B.Cu") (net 3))
 (segment locked (start 92.41 58.0) (end 93.41 57.0) (width 0.92) (layer "B.Cu") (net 3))
 (segment locked (start 93.41 57.0) (end 95.5 57.0) (width 0.92) (layer "B.Cu") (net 3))
 (segment locked (start 98.0 50.0) (end 98.0 42.5) (width 0.8) (layer "B.Cu") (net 3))
 (segment locked (start 98.0 42.5) (end 97.0 41.5) (width 0.8) (layer "B.Cu") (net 3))
 (segment locked (start 97.0 41.5) (end 70.5 41.5) (width 0.8) (layer "B.Cu") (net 3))
 (segment locked (start 57.9 41.5) (end 57.9 38.6) (width 0.92) (layer "B.Cu") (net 14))
 (segment locked (start 57.9 38.6) (end 56.94 37.56) (width 0.92) (layer "B.Cu") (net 14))
 (segment locked (start 56.94 37.56) (end 53.47 37.56) (width 0.92) (layer "B.Cu") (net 14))
 (segment locked (start 31.52 69.64) (end 31.52 76.6) (width 1.38) (layer "B.Cu") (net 17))
 (segment locked (start 31.52 76.6) (end 32.52 77.6) (width 1.38) (layer "B.Cu") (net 17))
 (segment locked (start 32.52 77.6) (end 104.6 77.6) (width 1.38) (layer "B.Cu") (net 17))
 (segment locked (start 104.6 77.6) (end 105.6 76.6) (width 1.38) (layer "B.Cu") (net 17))
 (segment locked (start 105.6 76.6) (end 105.6 70.24) (width 1.38) (layer "B.Cu") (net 17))
 (segment locked (start 67.97999999999999 35.379999999999995) (end 67.98 66.4) (width 0.92) (layer "B.Cu") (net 8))
 (segment locked (start 67.98 66.4) (end 68.98 67.4) (width 0.92) (layer "B.Cu") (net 8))
 (segment locked (start 68.98 67.4) (end 78.71 67.4) (width 0.92) (layer "B.Cu") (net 8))
 (segment locked (start 78.71 67.4) (end 79.71 66.4) (width 0.92) (layer "B.Cu") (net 8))
 (segment locked (start 79.71 66.4) (end 79.71 64.19) (width 0.92) (layer "B.Cu") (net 8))
 (segment locked (start 65.44 35.379999999999995) (end 65.44 68.4) (width 0.92) (layer "B.Cu") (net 9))
 (segment locked (start 65.44 68.4) (end 66.44 69.4) (width 0.92) (layer "B.Cu") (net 9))
 (segment locked (start 66.44 69.4) (end 81.25 69.4) (width 0.92) (layer "B.Cu") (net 9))
 (segment locked (start 81.25 69.4) (end 82.25 68.4) (width 0.92) (layer "B.Cu") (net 9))
 (segment locked (start 82.25 68.4) (end 82.25 64.19) (width 0.92) (layer "B.Cu") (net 9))
 (segment locked (start 105.6 60.08) (end 101.0 60.08) (width 0.92) (layer "B.Cu") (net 29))
 (segment locked (start 101.0 60.08) (end 100.0 61.08) (width 0.92) (layer "B.Cu") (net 29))
 (segment locked (start 100.0 61.08) (end 100.0 66.4) (width 0.92) (layer "B.Cu") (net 29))
 (segment locked (start 100.0 66.4) (end 99.0 67.4) (width 0.92) (layer "B.Cu") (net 29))
 (segment locked (start 99.0 67.4) (end 88.33 67.4) (width 0.92) (layer "B.Cu") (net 29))
 (segment locked (start 88.33 67.4) (end 87.33 66.4) (width 0.92) (layer "B.Cu") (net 29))
 (segment locked (start 87.33 66.4) (end 87.33 64.19) (width 0.92) (layer "B.Cu") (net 29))
 (segment locked (start 105.6 65.16) (end 102.6 65.16) (width 0.92) (layer "B.Cu") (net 28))
 (segment locked (start 102.6 65.16) (end 101.6 66.16) (width 0.92) (layer "B.Cu") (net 28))
 (segment locked (start 101.6 66.16) (end 101.6 68.4) (width 0.92) (layer "B.Cu") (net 28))
 (segment locked (start 101.6 68.4) (end 100.6 69.4) (width 0.92) (layer "B.Cu") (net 28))
 (segment locked (start 100.6 69.4) (end 85.79 69.4) (width 0.92) (layer "B.Cu") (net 28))
 (segment locked (start 85.79 69.4) (end 84.79 68.4) (width 0.92) (layer "B.Cu") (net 28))
 (segment locked (start 84.79 68.4) (end 84.79 64.19) (width 0.92) (layer "B.Cu") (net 28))
 (segment locked (start 90.84 35.379999999999995) (end 90.84 25.0) (width 0.92) (layer "B.Cu") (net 4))
 (segment locked (start 90.84 25.0) (end 89.84 24.0) (width 0.92) (layer "B.Cu") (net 4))
 (segment locked (start 89.84 24.0) (end 56.6 24.0) (width 0.92) (layer "B.Cu") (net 4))
 (segment locked (start 56.6 24.0) (end 55.6 23.0) (width 0.92) (layer "B.Cu") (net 4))
 (segment locked (start 55.6 23.0) (end 55.6 11.87) (width 0.92) (layer "B.Cu") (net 4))
 (segment locked (start 55.6 11.87) (end 54.6 10.87) (width 0.92) (layer "B.Cu") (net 4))
 (segment locked (start 54.6 10.87) (end 46.709999999999994 10.870000000000001) (width 0.92) (layer "B.Cu") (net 4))
 (segment locked (start 88.3 35.379999999999995) (end 88.3 27.0) (width 0.92) (layer "B.Cu") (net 5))
 (segment locked (start 88.3 27.0) (end 87.3 26.0) (width 0.92) (layer "B.Cu") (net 5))
 (segment locked (start 87.3 26.0) (end 54.6 26.0) (width 0.92) (layer "B.Cu") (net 5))
 (segment locked (start 54.6 26.0) (end 53.6 25.0) (width 0.92) (layer "B.Cu") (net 5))
 (segment locked (start 53.6 25.0) (end 53.6 14.41) (width 0.92) (layer "B.Cu") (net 5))
 (segment locked (start 53.6 14.41) (end 52.6 13.41) (width 0.92) (layer "B.Cu") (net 5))
 (segment locked (start 52.6 13.41) (end 46.709999999999994 13.41) (width 0.92) (layer "B.Cu") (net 5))
 (segment locked (start 85.75999999999999 35.379999999999995) (end 85.76 29.0) (width 0.92) (layer "B.Cu") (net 6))
 (segment locked (start 85.76 29.0) (end 84.76 28.0) (width 0.92) (layer "B.Cu") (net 6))
 (segment locked (start 84.76 28.0) (end 52.6 28.0) (width 0.92) (layer "B.Cu") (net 6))
 (segment locked (start 52.6 28.0) (end 51.6 27.0) (width 0.92) (layer "B.Cu") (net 6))
 (segment locked (start 51.6 27.0) (end 51.6 16.95) (width 0.92) (layer "B.Cu") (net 6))
 (segment locked (start 51.6 16.95) (end 50.6 15.95) (width 0.92) (layer "B.Cu") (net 6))
 (segment locked (start 50.6 15.95) (end 46.709999999999994 15.95) (width 0.92) (layer "B.Cu") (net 6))
 (segment locked (start 83.22 35.379999999999995) (end 83.22 31.0) (width 0.92) (layer "B.Cu") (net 7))
 (segment locked (start 83.22 31.0) (end 82.22 30.0) (width 0.92) (layer "B.Cu") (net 7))
 (segment locked (start 82.22 30.0) (end 50.6 30.0) (width 0.92) (layer "B.Cu") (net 7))
 (segment locked (start 50.6 30.0) (end 49.6 29.0) (width 0.92) (layer "B.Cu") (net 7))
 (segment locked (start 49.6 29.0) (end 49.6 19.49) (width 0.92) (layer "B.Cu") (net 7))
 (segment locked (start 49.6 19.49) (end 48.6 18.49) (width 0.92) (layer "B.Cu") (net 7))
 (segment locked (start 48.6 18.49) (end 46.709999999999994 18.490000000000002) (width 0.92) (layer "B.Cu") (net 7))
 (gr_line (start 0 0) (end 109.5 0) (layer "Edge.Cuts") (width 0.1))
 (gr_line (start 109.5 0) (end 109.5 85.5) (layer "Edge.Cuts") (width 0.1))
 (gr_line (start 109.5 85.5) (end 0 85.5) (layer "Edge.Cuts") (width 0.1))
 (gr_line (start 0 85.5) (end 0 0) (layer "Edge.Cuts") (width 0.1)))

